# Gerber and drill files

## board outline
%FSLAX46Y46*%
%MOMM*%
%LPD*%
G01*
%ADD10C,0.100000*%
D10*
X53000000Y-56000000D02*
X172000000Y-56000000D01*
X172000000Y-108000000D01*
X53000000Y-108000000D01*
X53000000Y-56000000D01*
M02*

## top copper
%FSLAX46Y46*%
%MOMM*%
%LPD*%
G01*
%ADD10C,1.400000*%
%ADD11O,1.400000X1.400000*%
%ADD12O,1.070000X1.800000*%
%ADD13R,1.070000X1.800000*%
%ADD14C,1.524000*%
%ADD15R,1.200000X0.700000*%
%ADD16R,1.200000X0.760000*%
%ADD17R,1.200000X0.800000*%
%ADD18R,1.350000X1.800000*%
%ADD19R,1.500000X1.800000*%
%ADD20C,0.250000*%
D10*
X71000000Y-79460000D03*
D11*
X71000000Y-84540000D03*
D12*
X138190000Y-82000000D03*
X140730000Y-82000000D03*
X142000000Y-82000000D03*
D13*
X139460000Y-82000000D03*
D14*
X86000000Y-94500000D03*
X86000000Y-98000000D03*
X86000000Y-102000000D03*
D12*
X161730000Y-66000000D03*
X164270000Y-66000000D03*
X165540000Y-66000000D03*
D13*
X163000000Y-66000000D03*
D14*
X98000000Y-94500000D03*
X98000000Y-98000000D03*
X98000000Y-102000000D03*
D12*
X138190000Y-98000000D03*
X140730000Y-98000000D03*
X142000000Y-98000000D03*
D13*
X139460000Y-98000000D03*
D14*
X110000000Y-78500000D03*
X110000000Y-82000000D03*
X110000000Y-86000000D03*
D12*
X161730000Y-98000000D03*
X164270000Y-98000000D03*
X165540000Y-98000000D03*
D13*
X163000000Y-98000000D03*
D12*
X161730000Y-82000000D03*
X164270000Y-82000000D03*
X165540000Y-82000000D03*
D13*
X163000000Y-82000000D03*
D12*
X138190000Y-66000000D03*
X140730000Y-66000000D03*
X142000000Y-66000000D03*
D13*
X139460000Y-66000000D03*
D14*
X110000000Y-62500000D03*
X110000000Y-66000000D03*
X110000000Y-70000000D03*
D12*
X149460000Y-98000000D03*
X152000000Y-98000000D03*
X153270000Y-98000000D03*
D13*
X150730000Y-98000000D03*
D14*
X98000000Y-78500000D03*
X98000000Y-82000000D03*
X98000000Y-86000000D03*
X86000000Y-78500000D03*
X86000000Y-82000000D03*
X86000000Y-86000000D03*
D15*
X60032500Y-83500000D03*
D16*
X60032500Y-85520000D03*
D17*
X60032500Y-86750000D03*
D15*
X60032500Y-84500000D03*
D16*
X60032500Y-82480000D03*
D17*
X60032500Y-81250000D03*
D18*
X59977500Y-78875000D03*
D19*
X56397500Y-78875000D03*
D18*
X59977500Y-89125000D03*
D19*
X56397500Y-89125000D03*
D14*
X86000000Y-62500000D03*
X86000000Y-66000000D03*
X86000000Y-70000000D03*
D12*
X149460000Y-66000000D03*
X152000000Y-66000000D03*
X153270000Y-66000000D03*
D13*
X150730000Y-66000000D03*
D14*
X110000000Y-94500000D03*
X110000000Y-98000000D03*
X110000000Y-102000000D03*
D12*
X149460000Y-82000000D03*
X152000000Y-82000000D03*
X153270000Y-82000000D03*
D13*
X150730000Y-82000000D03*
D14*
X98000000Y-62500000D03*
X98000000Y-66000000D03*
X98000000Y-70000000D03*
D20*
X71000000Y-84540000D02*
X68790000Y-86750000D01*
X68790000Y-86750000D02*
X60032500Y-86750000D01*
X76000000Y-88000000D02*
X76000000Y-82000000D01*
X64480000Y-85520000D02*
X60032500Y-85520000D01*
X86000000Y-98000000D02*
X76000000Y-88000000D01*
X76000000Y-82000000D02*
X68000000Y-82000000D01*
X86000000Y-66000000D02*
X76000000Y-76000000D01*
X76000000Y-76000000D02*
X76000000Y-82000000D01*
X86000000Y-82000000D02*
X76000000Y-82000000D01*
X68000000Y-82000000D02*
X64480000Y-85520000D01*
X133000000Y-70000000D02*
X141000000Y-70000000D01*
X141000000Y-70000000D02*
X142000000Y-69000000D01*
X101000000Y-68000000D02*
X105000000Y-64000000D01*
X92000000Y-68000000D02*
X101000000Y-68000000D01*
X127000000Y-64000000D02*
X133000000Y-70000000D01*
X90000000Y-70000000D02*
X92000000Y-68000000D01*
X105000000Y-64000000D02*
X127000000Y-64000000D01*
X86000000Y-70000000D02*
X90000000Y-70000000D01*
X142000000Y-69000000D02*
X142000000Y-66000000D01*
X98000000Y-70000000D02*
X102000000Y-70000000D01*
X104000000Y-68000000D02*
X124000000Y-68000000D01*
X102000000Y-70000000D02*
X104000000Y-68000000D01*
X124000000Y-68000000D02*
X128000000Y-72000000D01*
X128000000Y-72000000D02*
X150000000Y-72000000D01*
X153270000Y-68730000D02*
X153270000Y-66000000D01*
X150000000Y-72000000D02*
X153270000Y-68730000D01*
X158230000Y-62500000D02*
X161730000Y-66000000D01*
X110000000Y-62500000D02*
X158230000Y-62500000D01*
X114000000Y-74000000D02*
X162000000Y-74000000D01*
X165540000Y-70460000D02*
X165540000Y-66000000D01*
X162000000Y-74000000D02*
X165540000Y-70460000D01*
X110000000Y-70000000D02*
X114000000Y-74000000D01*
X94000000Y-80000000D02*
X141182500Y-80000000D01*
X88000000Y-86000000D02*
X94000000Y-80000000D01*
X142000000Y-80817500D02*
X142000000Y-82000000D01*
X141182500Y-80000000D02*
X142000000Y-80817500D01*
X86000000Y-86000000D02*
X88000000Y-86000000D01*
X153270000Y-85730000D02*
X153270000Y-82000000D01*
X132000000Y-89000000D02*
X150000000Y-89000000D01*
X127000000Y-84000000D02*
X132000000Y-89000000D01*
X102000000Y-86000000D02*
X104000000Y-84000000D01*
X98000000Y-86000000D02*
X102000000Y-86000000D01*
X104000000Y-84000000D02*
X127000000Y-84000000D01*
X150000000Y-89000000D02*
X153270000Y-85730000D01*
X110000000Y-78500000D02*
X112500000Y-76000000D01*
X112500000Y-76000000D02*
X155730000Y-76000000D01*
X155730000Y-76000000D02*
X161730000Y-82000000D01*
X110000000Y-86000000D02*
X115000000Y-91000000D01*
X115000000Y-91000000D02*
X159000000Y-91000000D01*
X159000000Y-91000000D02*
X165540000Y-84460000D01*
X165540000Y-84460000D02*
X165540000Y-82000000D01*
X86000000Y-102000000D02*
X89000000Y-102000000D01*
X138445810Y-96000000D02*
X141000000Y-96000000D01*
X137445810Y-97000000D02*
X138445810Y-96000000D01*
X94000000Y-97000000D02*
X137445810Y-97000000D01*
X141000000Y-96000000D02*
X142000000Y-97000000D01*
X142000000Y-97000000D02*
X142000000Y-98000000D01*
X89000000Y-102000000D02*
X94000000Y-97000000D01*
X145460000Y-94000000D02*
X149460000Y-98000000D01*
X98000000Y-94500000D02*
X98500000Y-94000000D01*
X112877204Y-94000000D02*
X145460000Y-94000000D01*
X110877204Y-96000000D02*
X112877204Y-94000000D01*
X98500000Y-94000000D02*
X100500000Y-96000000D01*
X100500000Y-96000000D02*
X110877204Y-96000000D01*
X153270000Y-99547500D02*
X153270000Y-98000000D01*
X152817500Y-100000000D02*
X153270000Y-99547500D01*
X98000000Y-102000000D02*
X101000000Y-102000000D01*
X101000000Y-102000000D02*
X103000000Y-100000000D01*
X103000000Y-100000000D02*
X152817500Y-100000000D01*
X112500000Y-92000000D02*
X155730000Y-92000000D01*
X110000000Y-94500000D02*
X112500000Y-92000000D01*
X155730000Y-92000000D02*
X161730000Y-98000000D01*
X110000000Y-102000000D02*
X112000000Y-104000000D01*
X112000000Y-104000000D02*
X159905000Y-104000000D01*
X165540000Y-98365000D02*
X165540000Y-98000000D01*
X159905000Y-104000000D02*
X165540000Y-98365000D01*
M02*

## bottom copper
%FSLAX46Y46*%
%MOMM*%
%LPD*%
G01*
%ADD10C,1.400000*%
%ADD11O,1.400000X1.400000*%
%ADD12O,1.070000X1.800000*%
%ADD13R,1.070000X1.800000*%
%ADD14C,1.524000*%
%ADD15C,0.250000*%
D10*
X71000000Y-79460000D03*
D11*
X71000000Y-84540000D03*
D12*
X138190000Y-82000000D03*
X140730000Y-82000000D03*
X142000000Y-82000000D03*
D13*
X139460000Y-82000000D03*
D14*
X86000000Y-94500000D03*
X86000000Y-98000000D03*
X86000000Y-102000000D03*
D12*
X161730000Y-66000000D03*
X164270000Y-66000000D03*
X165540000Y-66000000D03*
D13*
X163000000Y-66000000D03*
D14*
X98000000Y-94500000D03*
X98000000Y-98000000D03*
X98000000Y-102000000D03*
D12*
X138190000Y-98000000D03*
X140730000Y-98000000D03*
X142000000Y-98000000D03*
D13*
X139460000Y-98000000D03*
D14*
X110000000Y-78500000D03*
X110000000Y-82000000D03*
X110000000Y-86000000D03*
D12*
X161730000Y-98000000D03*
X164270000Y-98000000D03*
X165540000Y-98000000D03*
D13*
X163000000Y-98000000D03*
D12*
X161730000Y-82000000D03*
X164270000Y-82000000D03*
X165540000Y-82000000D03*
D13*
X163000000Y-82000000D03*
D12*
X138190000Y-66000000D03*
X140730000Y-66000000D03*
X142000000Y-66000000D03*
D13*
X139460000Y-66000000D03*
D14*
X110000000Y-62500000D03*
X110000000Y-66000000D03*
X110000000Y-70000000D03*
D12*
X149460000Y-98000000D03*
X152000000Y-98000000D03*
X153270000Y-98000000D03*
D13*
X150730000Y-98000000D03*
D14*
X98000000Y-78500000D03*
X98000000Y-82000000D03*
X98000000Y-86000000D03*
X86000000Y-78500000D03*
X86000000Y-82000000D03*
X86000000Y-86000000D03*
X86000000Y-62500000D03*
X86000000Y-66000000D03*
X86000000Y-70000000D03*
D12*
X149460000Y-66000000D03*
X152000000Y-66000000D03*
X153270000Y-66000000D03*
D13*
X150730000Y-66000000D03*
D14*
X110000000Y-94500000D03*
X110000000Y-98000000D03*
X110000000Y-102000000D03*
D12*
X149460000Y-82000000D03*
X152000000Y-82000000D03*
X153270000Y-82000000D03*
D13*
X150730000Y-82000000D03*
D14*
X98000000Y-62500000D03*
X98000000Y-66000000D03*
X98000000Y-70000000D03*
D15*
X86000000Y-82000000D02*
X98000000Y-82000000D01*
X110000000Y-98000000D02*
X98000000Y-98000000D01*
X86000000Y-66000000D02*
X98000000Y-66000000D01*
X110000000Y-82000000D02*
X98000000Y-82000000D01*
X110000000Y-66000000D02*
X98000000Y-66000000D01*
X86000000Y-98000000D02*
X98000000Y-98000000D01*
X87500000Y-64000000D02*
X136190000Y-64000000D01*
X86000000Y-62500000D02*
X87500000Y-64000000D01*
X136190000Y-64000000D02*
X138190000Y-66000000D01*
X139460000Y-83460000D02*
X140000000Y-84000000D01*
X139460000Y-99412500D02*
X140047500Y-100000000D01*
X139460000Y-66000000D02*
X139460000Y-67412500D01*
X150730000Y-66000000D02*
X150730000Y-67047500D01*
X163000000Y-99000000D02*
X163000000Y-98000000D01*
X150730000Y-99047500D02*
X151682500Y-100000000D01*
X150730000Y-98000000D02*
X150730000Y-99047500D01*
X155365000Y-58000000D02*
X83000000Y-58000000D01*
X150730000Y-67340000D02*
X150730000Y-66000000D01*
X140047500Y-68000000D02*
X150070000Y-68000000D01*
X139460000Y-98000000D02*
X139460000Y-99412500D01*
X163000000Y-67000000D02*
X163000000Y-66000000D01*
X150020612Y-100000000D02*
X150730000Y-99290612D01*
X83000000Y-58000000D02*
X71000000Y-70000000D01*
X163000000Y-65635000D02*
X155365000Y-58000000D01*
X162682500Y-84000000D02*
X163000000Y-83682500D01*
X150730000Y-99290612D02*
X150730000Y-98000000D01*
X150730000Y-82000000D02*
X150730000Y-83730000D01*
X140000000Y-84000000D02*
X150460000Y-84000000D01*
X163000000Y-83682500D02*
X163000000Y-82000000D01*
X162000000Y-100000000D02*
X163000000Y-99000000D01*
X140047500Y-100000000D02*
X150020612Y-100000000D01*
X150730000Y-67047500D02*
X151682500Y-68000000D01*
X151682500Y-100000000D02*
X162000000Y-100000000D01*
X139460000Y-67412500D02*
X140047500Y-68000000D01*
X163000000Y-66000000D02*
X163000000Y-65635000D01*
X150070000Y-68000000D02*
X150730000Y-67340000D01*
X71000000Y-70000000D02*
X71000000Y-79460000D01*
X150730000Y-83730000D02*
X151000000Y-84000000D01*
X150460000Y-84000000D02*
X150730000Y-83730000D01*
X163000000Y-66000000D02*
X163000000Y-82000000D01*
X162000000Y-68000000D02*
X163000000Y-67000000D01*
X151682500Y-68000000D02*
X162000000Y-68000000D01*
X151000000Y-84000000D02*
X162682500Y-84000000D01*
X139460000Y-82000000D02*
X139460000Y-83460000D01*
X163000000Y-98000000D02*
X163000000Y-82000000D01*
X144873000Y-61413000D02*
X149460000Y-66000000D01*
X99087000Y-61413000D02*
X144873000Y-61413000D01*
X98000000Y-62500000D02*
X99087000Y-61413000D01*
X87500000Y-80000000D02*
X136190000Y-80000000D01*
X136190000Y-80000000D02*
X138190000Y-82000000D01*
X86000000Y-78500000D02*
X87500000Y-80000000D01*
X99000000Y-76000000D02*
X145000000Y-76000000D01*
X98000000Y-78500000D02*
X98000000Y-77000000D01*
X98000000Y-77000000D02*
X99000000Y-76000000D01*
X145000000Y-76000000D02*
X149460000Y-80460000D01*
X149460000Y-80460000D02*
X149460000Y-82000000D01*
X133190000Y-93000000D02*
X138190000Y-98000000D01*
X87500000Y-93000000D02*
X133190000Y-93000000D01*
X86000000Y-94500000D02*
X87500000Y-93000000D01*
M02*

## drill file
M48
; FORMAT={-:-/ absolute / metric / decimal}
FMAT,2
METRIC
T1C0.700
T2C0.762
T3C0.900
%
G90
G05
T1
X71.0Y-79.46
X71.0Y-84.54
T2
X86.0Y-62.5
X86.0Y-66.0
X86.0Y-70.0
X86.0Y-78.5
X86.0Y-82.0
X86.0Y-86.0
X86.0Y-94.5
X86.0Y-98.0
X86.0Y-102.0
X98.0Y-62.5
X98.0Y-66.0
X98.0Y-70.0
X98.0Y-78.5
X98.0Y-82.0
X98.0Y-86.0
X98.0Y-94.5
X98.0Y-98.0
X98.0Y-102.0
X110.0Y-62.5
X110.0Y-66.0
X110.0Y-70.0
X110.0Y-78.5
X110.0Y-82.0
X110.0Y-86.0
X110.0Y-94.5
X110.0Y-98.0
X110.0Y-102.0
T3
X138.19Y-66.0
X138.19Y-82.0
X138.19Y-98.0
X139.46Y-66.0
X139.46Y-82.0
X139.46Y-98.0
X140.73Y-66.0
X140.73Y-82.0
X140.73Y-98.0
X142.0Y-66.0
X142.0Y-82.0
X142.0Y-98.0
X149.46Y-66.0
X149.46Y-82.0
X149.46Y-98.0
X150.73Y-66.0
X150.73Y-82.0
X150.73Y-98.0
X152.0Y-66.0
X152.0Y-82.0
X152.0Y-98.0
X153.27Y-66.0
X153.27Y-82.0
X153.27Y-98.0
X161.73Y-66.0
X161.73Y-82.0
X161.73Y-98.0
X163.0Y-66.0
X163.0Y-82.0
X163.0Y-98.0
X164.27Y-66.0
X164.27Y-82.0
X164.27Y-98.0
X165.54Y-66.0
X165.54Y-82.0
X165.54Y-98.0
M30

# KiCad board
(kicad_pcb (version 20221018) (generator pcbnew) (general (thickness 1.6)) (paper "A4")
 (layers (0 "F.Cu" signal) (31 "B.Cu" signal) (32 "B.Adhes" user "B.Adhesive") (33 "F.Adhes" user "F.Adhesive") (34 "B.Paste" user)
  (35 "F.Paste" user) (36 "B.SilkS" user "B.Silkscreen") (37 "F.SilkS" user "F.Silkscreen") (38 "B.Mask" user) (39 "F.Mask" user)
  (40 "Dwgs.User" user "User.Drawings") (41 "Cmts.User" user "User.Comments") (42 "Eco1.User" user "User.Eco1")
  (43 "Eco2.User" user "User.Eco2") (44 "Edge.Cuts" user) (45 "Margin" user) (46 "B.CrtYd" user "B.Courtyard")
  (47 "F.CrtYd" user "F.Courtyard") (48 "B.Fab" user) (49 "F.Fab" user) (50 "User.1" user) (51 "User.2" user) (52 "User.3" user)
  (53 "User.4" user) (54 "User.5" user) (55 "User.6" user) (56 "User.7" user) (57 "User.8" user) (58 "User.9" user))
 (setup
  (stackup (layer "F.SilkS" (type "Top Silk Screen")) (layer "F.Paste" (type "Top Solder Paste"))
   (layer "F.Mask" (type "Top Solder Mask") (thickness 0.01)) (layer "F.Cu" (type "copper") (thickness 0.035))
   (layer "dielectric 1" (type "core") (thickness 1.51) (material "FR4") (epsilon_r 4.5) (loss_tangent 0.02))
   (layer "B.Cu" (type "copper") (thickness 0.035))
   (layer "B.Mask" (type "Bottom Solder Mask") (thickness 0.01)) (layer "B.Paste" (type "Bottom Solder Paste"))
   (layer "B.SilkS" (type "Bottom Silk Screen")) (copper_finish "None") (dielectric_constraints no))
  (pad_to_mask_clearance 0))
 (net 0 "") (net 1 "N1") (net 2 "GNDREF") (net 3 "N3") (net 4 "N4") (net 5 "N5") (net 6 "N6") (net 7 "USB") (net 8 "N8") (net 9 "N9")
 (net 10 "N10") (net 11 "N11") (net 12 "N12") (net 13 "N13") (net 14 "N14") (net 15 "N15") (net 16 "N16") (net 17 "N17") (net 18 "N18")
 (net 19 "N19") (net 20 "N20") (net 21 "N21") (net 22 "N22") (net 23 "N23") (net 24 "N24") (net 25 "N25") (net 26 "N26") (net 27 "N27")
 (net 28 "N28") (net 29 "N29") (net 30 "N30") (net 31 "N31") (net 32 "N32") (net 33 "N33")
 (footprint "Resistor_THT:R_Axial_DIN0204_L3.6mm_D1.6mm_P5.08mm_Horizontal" (layer "F.Cu") (at 71 79.46 -90)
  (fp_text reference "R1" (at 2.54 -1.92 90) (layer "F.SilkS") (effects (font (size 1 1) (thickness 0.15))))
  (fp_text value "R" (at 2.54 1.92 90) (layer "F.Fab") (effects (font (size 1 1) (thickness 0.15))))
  (pad "1" thru_hole circle (at 0 0 270) (size 1.4 1.4) (drill 0.7) (layers "*.Cu" "*.Mask") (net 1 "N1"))
  (pad "2" thru_hole oval (at 5.08 0 270) (size 1.4 1.4) (drill 0.7) (layers "*.Cu" "*.Mask") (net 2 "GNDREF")))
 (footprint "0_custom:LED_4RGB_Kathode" (layer "F.Cu") (at 140.095 82)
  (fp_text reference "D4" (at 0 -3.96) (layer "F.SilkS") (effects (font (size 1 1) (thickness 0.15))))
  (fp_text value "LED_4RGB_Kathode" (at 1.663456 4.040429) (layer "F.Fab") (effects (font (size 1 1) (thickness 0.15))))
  (pad "1" thru_hole oval (at -1.905 0) (size 1.07 1.8) (drill 0.9) (layers "*.Cu" "*.Mask") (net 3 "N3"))
  (pad "2" thru_hole oval (at 0.635 0) (size 1.07 1.8) (drill 0.9) (layers "*.Cu" "*.Mask") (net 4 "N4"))
  (pad "3" thru_hole oval (at 1.905 0) (size 1.07 1.8) (drill 0.9) (layers "*.Cu" "*.Mask") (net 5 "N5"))
  (pad "4" thru_hole rect (at -0.635 0) (size 1.07 1.8) (drill 0.9) (layers "*.Cu" "*.Mask") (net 1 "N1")))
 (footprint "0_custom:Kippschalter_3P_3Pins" (layer "F.Cu") (at 86 98 -90)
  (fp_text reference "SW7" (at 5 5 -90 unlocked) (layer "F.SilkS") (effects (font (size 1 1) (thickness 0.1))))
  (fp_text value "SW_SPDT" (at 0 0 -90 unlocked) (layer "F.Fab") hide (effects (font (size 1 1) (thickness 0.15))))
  (pad "1" thru_hole circle (at -3.5 0 270) (size 1.524 1.524) (drill 0.762) (layers "*.Cu" "*.Mask") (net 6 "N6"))
  (pad "2" thru_hole circle (at 0 0 270) (size 1.524 1.524) (drill 0.762) (layers "*.Cu" "*.Mask") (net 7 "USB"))
  (pad "3" thru_hole circle (at 4 0 270) (size 1.524 1.524) (drill 0.762) (layers "*.Cu" "*.Mask") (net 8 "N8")))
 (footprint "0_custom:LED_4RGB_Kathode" (layer "F.Cu") (at 163.635 66)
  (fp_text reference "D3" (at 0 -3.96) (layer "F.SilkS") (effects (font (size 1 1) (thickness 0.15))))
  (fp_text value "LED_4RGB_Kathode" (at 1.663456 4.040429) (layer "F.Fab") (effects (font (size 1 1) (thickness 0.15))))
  (pad "1" thru_hole oval (at -1.905 0) (size 1.07 1.8) (drill 0.9) (layers "*.Cu" "*.Mask") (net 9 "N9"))
  (pad "2" thru_hole oval (at 0.635 0) (size 1.07 1.8) (drill 0.9) (layers "*.Cu" "*.Mask") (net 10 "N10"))
  (pad "3" thru_hole oval (at 1.905 0) (size 1.07 1.8) (drill 0.9) (layers "*.Cu" "*.Mask") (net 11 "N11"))
  (pad "4" thru_hole rect (at -0.635 0) (size 1.07 1.8) (drill 0.9) (layers "*.Cu" "*.Mask") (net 1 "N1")))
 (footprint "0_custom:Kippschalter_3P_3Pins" (layer "F.Cu") (at 98 98 -90)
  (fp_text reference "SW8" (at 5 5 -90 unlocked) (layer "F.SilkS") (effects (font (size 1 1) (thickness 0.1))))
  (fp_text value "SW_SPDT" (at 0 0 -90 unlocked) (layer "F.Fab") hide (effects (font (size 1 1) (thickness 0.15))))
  (pad "1" thru_hole circle (at -3.5 0 270) (size 1.524 1.524) (drill 0.762) (layers "*.Cu" "*.Mask") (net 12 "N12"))
  (pad "2" thru_hole circle (at 0 0 270) (size 1.524 1.524) (drill 0.762) (layers "*.Cu" "*.Mask") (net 7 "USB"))
  (pad "3" thru_hole circle (at 4 0 270) (size 1.524 1.524) (drill 0.762) (layers "*.Cu" "*.Mask") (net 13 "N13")))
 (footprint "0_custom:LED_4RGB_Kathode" (layer "F.Cu") (at 140.095 98)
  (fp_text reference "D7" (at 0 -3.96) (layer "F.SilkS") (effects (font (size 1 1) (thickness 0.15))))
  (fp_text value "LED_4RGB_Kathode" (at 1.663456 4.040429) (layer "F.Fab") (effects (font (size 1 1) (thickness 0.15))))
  (pad "1" thru_hole oval (at -1.905 0) (size 1.07 1.8) (drill 0.9) (layers "*.Cu" "*.Mask") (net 6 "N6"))
  (pad "2" thru_hole oval (at 0.635 0) (size 1.07 1.8) (drill 0.9) (layers "*.Cu" "*.Mask") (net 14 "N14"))
  (pad "3" thru_hole oval (at 1.905 0) (size 1.07 1.8) (drill 0.9) (layers "*.Cu" "*.Mask") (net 8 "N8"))
  (pad "4" thru_hole rect (at -0.635 0) (size 1.07 1.8) (drill 0.9) (layers "*.Cu" "*.Mask") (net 1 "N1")))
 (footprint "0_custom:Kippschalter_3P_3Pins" (layer "F.Cu") (at 110 82 -90)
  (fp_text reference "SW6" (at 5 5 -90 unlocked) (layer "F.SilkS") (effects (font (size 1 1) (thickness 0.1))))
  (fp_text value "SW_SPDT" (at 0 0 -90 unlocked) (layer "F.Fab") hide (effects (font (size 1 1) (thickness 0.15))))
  (pad "1" thru_hole circle (at -3.5 0 270) (size 1.524 1.524) (drill 0.762) (layers "*.Cu" "*.Mask") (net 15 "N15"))
  (pad "2" thru_hole circle (at 0 0 270) (size 1.524 1.524) (drill 0.762) (layers "*.Cu" "*.Mask") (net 7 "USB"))
  (pad "3" thru_hole circle (at 4 0 270) (size 1.524 1.524) (drill 0.762) (layers "*.Cu" "*.Mask") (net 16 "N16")))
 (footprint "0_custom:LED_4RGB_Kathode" (layer "F.Cu") (at 163.635 98)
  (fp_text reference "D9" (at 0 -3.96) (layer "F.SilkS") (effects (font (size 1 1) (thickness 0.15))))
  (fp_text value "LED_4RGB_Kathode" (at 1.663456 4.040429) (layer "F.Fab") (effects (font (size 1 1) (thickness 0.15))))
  (pad "1" thru_hole oval (at -1.905 0) (size 1.07 1.8) (drill 0.9) (layers "*.Cu" "*.Mask") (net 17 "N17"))
  (pad "2" thru_hole oval (at 0.635 0) (size 1.07 1.8) (drill 0.9) (layers "*.Cu" "*.Mask") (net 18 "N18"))
  (pad "3" thru_hole oval (at 1.905 0) (size 1.07 1.8) (drill 0.9) (layers "*.Cu" "*.Mask") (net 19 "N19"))
  (pad "4" thru_hole rect (at -0.635 0) (size 1.07 1.8) (drill 0.9) (layers "*.Cu" "*.Mask") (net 1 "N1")))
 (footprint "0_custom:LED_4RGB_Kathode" (layer "F.Cu") (at 163.635 82)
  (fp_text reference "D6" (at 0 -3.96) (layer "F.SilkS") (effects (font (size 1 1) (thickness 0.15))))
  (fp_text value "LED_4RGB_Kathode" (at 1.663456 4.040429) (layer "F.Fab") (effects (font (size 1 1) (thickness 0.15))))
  (pad "1" thru_hole oval (at -1.905 0) (size 1.07 1.8) (drill 0.9) (layers "*.Cu" "*.Mask") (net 15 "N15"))
  (pad "2" thru_hole oval (at 0.635 0) (size 1.07 1.8) (drill 0.9) (layers "*.Cu" "*.Mask") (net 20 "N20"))
  (pad "3" thru_hole oval (at 1.905 0) (size 1.07 1.8) (drill 0.9) (layers "*.Cu" "*.Mask") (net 16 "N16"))
  (pad "4" thru_hole rect (at -0.635 0) (size 1.07 1.8) (drill 0.9) (layers "*.Cu" "*.Mask") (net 1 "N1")))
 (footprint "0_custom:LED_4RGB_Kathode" (layer "F.Cu") (at 140.095 66)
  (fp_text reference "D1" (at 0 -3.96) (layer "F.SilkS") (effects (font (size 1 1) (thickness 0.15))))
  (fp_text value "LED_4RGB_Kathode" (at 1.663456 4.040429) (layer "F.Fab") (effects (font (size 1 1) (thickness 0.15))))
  (pad "1" thru_hole oval (at -1.905 0) (size 1.07 1.8) (drill 0.9) (layers "*.Cu" "*.Mask") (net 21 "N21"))
  (pad "2" thru_hole oval (at 0.635 0) (size 1.07 1.8) (drill 0.9) (layers "*.Cu" "*.Mask") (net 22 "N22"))
  (pad "3" thru_hole oval (at 1.905 0) (size 1.07 1.8) (drill 0.9) (layers "*.Cu" "*.Mask") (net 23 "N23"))
  (pad "4" thru_hole rect (at -0.635 0) (size 1.07 1.8) (drill 0.9) (layers "*.Cu" "*.Mask") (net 1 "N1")))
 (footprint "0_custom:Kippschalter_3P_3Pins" (layer "F.Cu") (at 110 66 -90)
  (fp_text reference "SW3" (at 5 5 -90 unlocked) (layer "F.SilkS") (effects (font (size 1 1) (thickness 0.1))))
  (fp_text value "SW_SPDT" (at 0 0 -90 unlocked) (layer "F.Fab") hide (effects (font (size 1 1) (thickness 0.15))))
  (pad "1" thru_hole circle (at -3.5 0 270) (size 1.524 1.524) (drill 0.762) (layers "*.Cu" "*.Mask") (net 9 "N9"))
  (pad "2" thru_hole circle (at 0 0 270) (size 1.524 1.524) (drill 0.762) (layers "*.Cu" "*.Mask") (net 7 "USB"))
  (pad "3" thru_hole circle (at 4 0 270) (size 1.524 1.524) (drill 0.762) (layers "*.Cu" "*.Mask") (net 11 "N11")))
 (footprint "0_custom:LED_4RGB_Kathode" (layer "F.Cu") (at 151.365 98)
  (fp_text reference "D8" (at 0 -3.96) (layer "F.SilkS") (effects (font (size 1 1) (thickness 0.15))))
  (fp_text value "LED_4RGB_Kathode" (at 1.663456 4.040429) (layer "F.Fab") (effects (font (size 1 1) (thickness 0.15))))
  (pad "1" thru_hole oval (at -1.905 0) (size 1.07 1.8) (drill 0.9) (layers "*.Cu" "*.Mask") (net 12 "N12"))
  (pad "2" thru_hole oval (at 0.635 0) (size 1.07 1.8) (drill 0.9) (layers "*.Cu" "*.Mask") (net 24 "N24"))
  (pad "3" thru_hole oval (at 1.905 0) (size 1.07 1.8) (drill 0.9) (layers "*.Cu" "*.Mask") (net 13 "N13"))
  (pad "4" thru_hole rect (at -0.635 0) (size 1.07 1.8) (drill 0.9) (layers "*.Cu" "*.Mask") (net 1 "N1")))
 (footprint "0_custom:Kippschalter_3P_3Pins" (layer "F.Cu") (at 98 82 -90)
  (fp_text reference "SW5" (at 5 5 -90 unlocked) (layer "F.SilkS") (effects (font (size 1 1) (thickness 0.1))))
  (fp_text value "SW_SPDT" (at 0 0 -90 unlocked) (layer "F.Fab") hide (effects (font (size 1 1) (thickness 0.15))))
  (pad "1" thru_hole circle (at -3.5 0 270) (size 1.524 1.524) (drill 0.762) (layers "*.Cu" "*.Mask") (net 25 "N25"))
  (pad "2" thru_hole circle (at 0 0 270) (size 1.524 1.524) (drill 0.762) (layers "*.Cu" "*.Mask") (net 7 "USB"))
  (pad "3" thru_hole circle (at 4 0 270) (size 1.524 1.524) (drill 0.762) (layers "*.Cu" "*.Mask") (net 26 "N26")))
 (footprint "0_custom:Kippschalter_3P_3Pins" (layer "F.Cu") (at 86 82 -90)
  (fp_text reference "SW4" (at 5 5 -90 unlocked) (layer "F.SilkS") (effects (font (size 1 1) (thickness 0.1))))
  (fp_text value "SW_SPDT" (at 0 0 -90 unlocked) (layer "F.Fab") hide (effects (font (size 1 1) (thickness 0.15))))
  (pad "1" thru_hole circle (at -3.5 0 270) (size 1.524 1.524) (drill 0.762) (layers "*.Cu" "*.Mask") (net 3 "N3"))
  (pad "2" thru_hole circle (at 0 0 270) (size 1.524 1.524) (drill 0.762) (layers "*.Cu" "*.Mask") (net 7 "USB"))
  (pad "3" thru_hole circle (at 4 0 270) (size 1.524 1.524) (drill 0.762) (layers "*.Cu" "*.Mask") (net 5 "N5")))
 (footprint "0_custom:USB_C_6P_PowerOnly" (layer "F.Cu") (at 57 84 -90)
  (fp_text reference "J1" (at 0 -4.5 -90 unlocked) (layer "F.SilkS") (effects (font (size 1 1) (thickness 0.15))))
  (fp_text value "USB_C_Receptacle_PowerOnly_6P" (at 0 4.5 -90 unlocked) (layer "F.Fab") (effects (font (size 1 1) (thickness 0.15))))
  (pad "A5" smd rect (at -0.5 -3.0325 270) (size 0.7 1.2) (layers "F.Cu" "F.Paste" "F.Mask") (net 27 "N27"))
  (pad "A9" smd rect (at 1.52 -3.0325 90) (size 0.76 1.2) (layers "F.Cu" "F.Paste" "F.Mask") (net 7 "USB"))
  (pad "A12" smd rect (at 2.75 -3.0325 90) (size 0.8 1.2) (layers "F.Cu" "F.Paste" "F.Mask") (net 2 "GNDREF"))
  (pad "B5" smd rect (at 0.5 -3.0325 90) (size 0.7 1.2) (layers "F.Cu" "F.Paste" "F.Mask") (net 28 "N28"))
  (pad "B9" smd rect (at -1.52 -3.0325 270) (size 0.76 1.2) (layers "F.Cu" "F.Paste" "F.Mask") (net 7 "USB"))
  (pad "B12" smd rect (at -2.75 -3.0325 270) (size 0.8 1.2) (layers "F.Cu" "F.Paste" "F.Mask") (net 2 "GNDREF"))
  (pad "S1" smd rect (at -5.125 -2.9775 270) (size 1.8 1.35) (layers "F.Cu" "F.Paste" "F.Mask") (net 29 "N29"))
  (pad "S1" smd rect (at -5.125 0.6025 270) (size 1.8 1.5) (layers "F.Cu" "F.Paste" "F.Mask") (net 29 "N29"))
  (pad "S1" smd rect (at 5.125 -2.9775 270) (size 1.8 1.35) (layers "F.Cu" "F.Paste" "F.Mask") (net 29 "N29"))
  (pad "S1" smd rect (at 5.125 0.6025 270) (size 1.8 1.5) (layers "F.Cu" "F.Paste" "F.Mask") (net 29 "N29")))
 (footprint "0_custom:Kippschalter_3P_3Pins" (layer "F.Cu") (at 86 66 -90)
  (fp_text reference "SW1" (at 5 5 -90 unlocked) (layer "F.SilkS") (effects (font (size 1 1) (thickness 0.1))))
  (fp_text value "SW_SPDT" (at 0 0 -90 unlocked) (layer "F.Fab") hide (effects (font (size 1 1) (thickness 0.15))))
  (pad "1" thru_hole circle (at -3.5 0 270) (size 1.524 1.524) (drill 0.762) (layers "*.Cu" "*.Mask") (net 21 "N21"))
  (pad "2" thru_hole circle (at 0 0 270) (size 1.524 1.524) (drill 0.762) (layers "*.Cu" "*.Mask") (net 7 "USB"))
  (pad "3" thru_hole circle (at 4 0 270) (size 1.524 1.524) (drill 0.762) (layers "*.Cu" "*.Mask") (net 23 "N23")))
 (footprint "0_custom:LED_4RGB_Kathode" (layer "F.Cu") (at 151.365 66)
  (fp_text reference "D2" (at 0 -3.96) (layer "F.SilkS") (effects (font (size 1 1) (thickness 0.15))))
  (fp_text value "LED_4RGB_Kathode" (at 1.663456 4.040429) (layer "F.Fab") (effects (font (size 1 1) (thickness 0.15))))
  (pad "1" thru_hole oval (at -1.905 0) (size 1.07 1.8) (drill 0.9) (layers "*.Cu" "*.Mask") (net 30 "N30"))
  (pad "2" thru_hole oval (at 0.635 0) (size 1.07 1.8) (drill 0.9) (layers "*.Cu" "*.Mask") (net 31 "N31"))
  (pad "3" thru_hole oval (at 1.905 0) (size 1.07 1.8) (drill 0.9) (layers "*.Cu" "*.Mask") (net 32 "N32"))
  (pad "4" thru_hole rect (at -0.635 0) (size 1.07 1.8) (drill 0.9) (layers "*.Cu" "*.Mask") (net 1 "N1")))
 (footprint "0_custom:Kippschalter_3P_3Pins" (layer "F.Cu") (at 110 98 -90)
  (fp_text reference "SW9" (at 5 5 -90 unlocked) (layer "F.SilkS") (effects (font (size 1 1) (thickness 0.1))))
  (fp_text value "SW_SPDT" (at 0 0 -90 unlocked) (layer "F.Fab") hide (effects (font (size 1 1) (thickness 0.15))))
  (pad "1" thru_hole circle (at -3.5 0 270) (size 1.524 1.524) (drill 0.762) (layers "*.Cu" "*.Mask") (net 17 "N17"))
  (pad "2" thru_hole circle (at 0 0 270) (size 1.524 1.524) (drill 0.762) (layers "*.Cu" "*.Mask") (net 7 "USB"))
  (pad "3" thru_hole circle (at 4 0 270) (size 1.524 1.524) (drill 0.762) (layers "*.Cu" "*.Mask") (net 19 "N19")))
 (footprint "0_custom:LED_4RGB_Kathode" (layer "F.Cu") (at 151.365 82)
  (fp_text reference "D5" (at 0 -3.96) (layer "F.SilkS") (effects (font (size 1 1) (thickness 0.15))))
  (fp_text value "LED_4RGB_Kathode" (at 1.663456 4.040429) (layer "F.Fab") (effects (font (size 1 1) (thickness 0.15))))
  (pad "1" thru_hole oval (at -1.905 0) (size 1.07 1.8) (drill 0.9) (layers "*.Cu" "*.Mask") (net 25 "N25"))
  (pad "2" thru_hole oval (at 0.635 0) (size 1.07 1.8) (drill 0.9) (layers "*.Cu" "*.Mask") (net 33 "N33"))
  (pad "3" thru_hole oval (at 1.905 0) (size 1.07 1.8) (drill 0.9) (layers "*.Cu" "*.Mask") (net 26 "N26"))
  (pad "4" thru_hole rect (at -0.635 0) (size 1.07 1.8) (drill 0.9) (layers "*.Cu" "*.Mask") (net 1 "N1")))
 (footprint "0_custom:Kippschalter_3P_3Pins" (layer "F.Cu") (at 98 66 -90)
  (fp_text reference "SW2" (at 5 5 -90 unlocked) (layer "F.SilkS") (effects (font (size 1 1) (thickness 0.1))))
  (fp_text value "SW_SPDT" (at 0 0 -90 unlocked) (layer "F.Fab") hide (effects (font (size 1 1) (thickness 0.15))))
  (pad "1" thru_hole circle (at -3.5 0 270) (size 1.524 1.524) (drill 0.762) (layers "*.Cu" "*.Mask") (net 30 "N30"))
  (pad "2" thru_hole circle (at 0 0 270) (size 1.524 1.524) (drill 0.762) (layers "*.Cu" "*.Mask") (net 7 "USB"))
  (pad "3" thru_hole circle (at 4 0 270) (size 1.524 1.524) (drill 0.762) (layers "*.Cu" "*.Mask") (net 32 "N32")))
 (gr_rect (start 53 56) (end 172 108) (stroke (width 0.1) (type default)) (fill none) (layer "Edge.Cuts"))
 (segment (start 71 84.54) (end 68.79 86.75) (width 0.25) (layer "F.Cu") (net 2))
 (segment (start 68.79 86.75) (end 60.0325 86.75) (width 0.25) (layer "F.Cu") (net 2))
 (segment (start 76 88) (end 76 82) (width 0.25) (layer "F.Cu") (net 7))
 (segment (start 64.48 85.52) (end 60.0325 85.52) (width 0.25) (layer "F.Cu") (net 7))
 (segment (start 86 98) (end 76 88) (width 0.25) (layer "F.Cu") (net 7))
 (segment (start 76 82) (end 68 82) (width 0.25) (layer "F.Cu") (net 7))
 (segment (start 86 66) (end 76 76) (width 0.25) (layer "F.Cu") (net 7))
 (segment (start 76 76) (end 76 82) (width 0.25) (layer "F.Cu") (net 7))
 (segment (start 86 82) (end 76 82) (width 0.25) (layer "F.Cu") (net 7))
 (segment (start 68 82) (end 64.48 85.52) (width 0.25) (layer "F.Cu") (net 7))
 (segment (start 86 82) (end 98 82) (width 0.25) (layer "B.Cu") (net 7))
 (segment (start 110 98) (end 98 98) (width 0.25) (layer "B.Cu") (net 7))
 (segment (start 86 66) (end 98 66) (width 0.25) (layer "B.Cu") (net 7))
 (segment (start 110 82) (end 98 82) (width 0.25) (layer "B.Cu") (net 7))
 (segment (start 110 66) (end 98 66) (width 0.25) (layer "B.Cu") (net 7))
 (segment (start 86 98) (end 98 98) (width 0.25) (layer "B.Cu") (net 7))
 (segment (start 87.5 64) (end 136.19 64) (width 0.25) (layer "B.Cu") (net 21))
 (segment (start 86 62.5) (end 87.5 64) (width 0.25) (layer "B.Cu") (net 21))
 (segment (start 136.19 64) (end 138.19 66) (width 0.25) (layer "B.Cu") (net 21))
 (segment (start 133 70) (end 141 70) (width 0.25) (layer "F.Cu") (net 23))
 (segment (start 141 70) (end 142 69) (width 0.25) (layer "F.Cu") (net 23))
 (segment (start 101 68) (end 105 64) (width 0.25) (layer "F.Cu") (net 23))
 (segment (start 92 68) (end 101 68) (width 0.25) (layer "F.Cu") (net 23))
 (segment (start 127 64) (end 133 70) (width 0.25) (layer "F.Cu") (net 23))
 (segment (start 90 70) (end 92 68) (width 0.25) (layer "F.Cu") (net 23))
 (segment (start 105 64) (end 127 64) (width 0.25) (layer "F.Cu") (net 23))
 (segment (start 86 70) (end 90 70) (width 0.25) (layer "F.Cu") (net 23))
 (segment (start 142 69) (end 142 66) (width 0.25) (layer "F.Cu") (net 23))
 (segment (start 139.46 83.46) (end 140 84) (width 0.25) (layer "B.Cu") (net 1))
 (segment (start 139.46 99.4125) (end 140.0475 100) (width 0.25) (layer "B.Cu") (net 1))
 (segment (start 139.46 66) (end 139.46 67.4125) (width 0.25) (layer "B.Cu") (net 1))
 (segment (start 150.73 66) (end 150.73 67.0475) (width 0.25) (layer "B.Cu") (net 1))
 (segment (start 163 99) (end 163 98) (width 0.25) (layer "B.Cu") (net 1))
 (segment (start 150.73 99.0475) (end 151.6825 100) (width 0.25) (layer "B.Cu") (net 1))
 (segment (start 150.73 98) (end 150.73 99.0475) (width 0.25) (layer "B.Cu") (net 1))
 (segment (start 155.365 58) (end 83 58) (width 0.25) (layer "B.Cu") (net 1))
 (segment (start 150.73 67.34) (end 150.73 66) (width 0.25) (layer "B.Cu") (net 1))
 (segment (start 140.0475 68) (end 150.07 68) (width 0.25) (layer "B.Cu") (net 1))
 (segment (start 139.46 98) (end 139.46 99.4125) (width 0.25) (layer "B.Cu") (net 1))
 (segment (start 163 67) (end 163 66) (width 0.25) (layer "B.Cu") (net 1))
 (segment (start 150.020612 100) (end 150.73 99.290612) (width 0.25) (layer "B.Cu") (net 1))
 (segment (start 83 58) (end 71 70) (width 0.25) (layer "B.Cu") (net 1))
 (segment (start 163 65.635) (end 155.365 58) (width 0.25) (layer "B.Cu") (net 1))
 (segment (start 162.6825 84) (end 163 83.6825) (width 0.25) (layer "B.Cu") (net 1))
 (segment (start 150.73 99.290612) (end 150.73 98) (width 0.25) (layer "B.Cu") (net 1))
 (segment (start 150.73 82) (end 150.73 83.73) (width 0.25) (layer "B.Cu") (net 1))
 (segment (start 140 84) (end 150.46 84) (width 0.25) (layer "B.Cu") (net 1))
 (segment (start 163 83.6825) (end 163 82) (width 0.25) (layer "B.Cu") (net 1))
 (segment (start 162 100) (end 163 99) (width 0.25) (layer "B.Cu") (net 1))
 (segment (start 140.0475 100) (end 150.020612 100) (width 0.25) (layer "B.Cu") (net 1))
 (segment (start 150.73 67.0475) (end 151.6825 68) (width 0.25) (layer "B.Cu") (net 1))
 (segment (start 151.6825 100) (end 162 100) (width 0.25) (layer "B.Cu") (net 1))
 (segment (start 139.46 67.4125) (end 140.0475 68) (width 0.25) (layer "B.Cu") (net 1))
 (segment (start 163 66) (end 163 65.635) (width 0.25) (layer "B.Cu") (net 1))
 (segment (start 150.07 68) (end 150.73 67.34) (width 0.25) (layer "B.Cu") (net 1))
 (segment (start 71 70) (end 71 79.46) (width 0.25) (layer "B.Cu") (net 1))
 (segment (start 150.73 83.73) (end 151 84) (width 0.25) (layer "B.Cu") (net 1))
 (segment (start 150.46 84) (end 150.73 83.73) (width 0.25) (layer "B.Cu") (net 1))
 (segment (start 163 66) (end 163 82) (width 0.25) (layer "B.Cu") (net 1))
 (segment (start 162 68) (end 163 67) (width 0.25) (layer "B.Cu") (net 1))
 (segment (start 151.6825 68) (end 162 68) (width 0.25) (layer "B.Cu") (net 1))
 (segment (start 151 84) (end 162.6825 84) (width 0.25) (layer "B.Cu") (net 1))
 (segment (start 139.46 82) (end 139.46 83.46) (width 0.25) (layer "B.Cu") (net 1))
 (segment (start 163 98) (end 163 82) (width 0.25) (layer "B.Cu") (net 1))
 (segment (start 144.873 61.413) (end 149.46 66) (width 0.25) (layer "B.Cu") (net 30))
 (segment (start 99.087 61.413) (end 144.873 61.413) (width 0.25) (layer "B.Cu") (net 30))
 (segment (start 98 62.5) (end 99.087 61.413) (width 0.25) (layer "B.Cu") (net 30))
 (segment (start 98 70) (end 102 70) (width 0.25) (layer "F.Cu") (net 32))
 (segment (start 104 68) (end 124 68) (width 0.25) (layer "F.Cu") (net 32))
 (segment (start 102 70) (end 104 68) (width 0.25) (layer "F.Cu") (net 32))
 (segment (start 124 68) (end 128 72) (width 0.25) (layer "F.Cu") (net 32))
 (segment (start 128 72) (end 150 72) (width 0.25) (layer "F.Cu") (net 32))
 (segment (start 153.27 68.73) (end 153.27 66) (width 0.25) (layer "F.Cu") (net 32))
 (segment (start 150 72) (end 153.27 68.73) (width 0.25) (layer "F.Cu") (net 32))
 (segment (start 158.23 62.5) (end 161.73 66) (width 0.25) (layer "F.Cu") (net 9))
 (segment (start 110 62.5) (end 158.23 62.5) (width 0.25) (layer "F.Cu") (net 9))
 (segment (start 114 74) (end 162 74) (width 0.25) (layer "F.Cu") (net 11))
 (segment (start 165.54 70.46) (end 165.54 66) (width 0.25) (layer "F.Cu") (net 11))
 (segment (start 162 74) (end 165.54 70.46) (width 0.25) (layer "F.Cu") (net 11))
 (segment (start 110 70) (end 114 74) (width 0.25) (layer "F.Cu") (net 11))
 (segment (start 87.5 80) (end 136.19 80) (width 0.25) (layer "B.Cu") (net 3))
 (segment (start 136.19 80) (end 138.19 82) (width 0.25) (layer "B.Cu") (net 3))
 (segment (start 86 78.5) (end 87.5 80) (width 0.25) (layer "B.Cu") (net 3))
 (segment (start 94 80) (end 141.1825 80) (width 0.25) (layer "F.Cu") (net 5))
 (segment (start 88 86) (end 94 80) (width 0.25) (layer "F.Cu") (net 5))
 (segment (start 142 80.8175) (end 142 82) (width 0.25) (layer "F.Cu") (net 5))
 (segment (start 141.1825 80) (end 142 80.8175) (width 0.25) (layer "F.Cu") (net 5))
 (segment (start 86 86) (end 88 86) (width 0.25) (layer "F.Cu") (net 5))
 (segment (start 99 76) (end 145 76) (width 0.25) (layer "B.Cu") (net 25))
 (segment (start 98 78.5) (end 98 77) (width 0.25) (layer "B.Cu") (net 25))
 (segment (start 98 77) (end 99 76) (width 0.25) (layer "B.Cu") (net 25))
 (segment (start 145 76) (end 149.46 80.46) (width 0.25) (layer "B.Cu") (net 25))
 (segment (start 149.46 80.46) (end 149.46 82) (width 0.25) (layer "B.Cu") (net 25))
 (segment (start 153.27 85.73) (end 153.27 82) (width 0.25) (layer "F.Cu") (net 26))
 (segment (start 132 89) (end 150 89) (width 0.25) (layer "F.Cu") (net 26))
 (segment (start 127 84) (end 132 89) (width 0.25) (layer "F.Cu") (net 26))
 (segment (start 102 86) (end 104 84) (width 0.25) (layer "F.Cu") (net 26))
 (segment (start 98 86) (end 102 86) (width 0.25) (layer "F.Cu") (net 26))
 (segment (start 104 84) (end 127 84) (width 0.25) (layer "F.Cu") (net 26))
 (segment (start 150 89) (end 153.27 85.73) (width 0.25) (layer "F.Cu") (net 26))
 (segment (start 110 78.5) (end 112.5 76) (width 0.25) (layer "F.Cu") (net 15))
 (segment (start 112.5 76) (end 155.73 76) (width 0.25) (layer "F.Cu") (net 15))
 (segment (start 155.73 76) (end 161.73 82) (width 0.25) (layer "F.Cu") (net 15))
 (segment (start 110 86) (end 115 91) (width 0.25) (layer "F.Cu") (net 16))
 (segment (start 115 91) (end 159 91) (width 0.25) (layer "F.Cu") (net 16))
 (segment (start 159 91) (end 165.54 84.46) (width 0.25) (layer "F.Cu") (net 16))
 (segment (start 165.54 84.46) (end 165.54 82) (width 0.25) (layer "F.Cu") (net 16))
 (segment (start 133.19 93) (end 138.19 98) (width 0.25) (layer "B.Cu") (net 6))
 (segment (start 87.5 93) (end 133.19 93) (width 0.25) (layer "B.Cu") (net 6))
 (segment (start 86 94.5) (end 87.5 93) (width 0.25) (layer "B.Cu") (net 6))
 (segment (start 86 102) (end 89 102) (width 0.25) (layer "F.Cu") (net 8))
 (segment (start 138.44581 96) (end 141 96) (width 0.25) (layer "F.Cu") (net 8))
 (segment (start 137.44581 97) (end 138.44581 96) (width 0.25) (layer "F.Cu") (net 8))
 (segment (start 94 97) (end 137.44581 97) (width 0.25) (layer "F.Cu") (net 8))
 (segment (start 141 96) (end 142 97) (width 0.25) (layer "F.Cu") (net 8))
 (segment (start 142 97) (end 142 98) (width 0.25) (layer "F.Cu") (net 8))
 (segment (start 89 102) (end 94 97) (width 0.25) (layer "F.Cu") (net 8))
 (segment (start 145.46 94) (end 149.46 98) (width 0.25) (layer "F.Cu") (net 12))
 (segment (start 98 94.5) (end 98.5 94) (width 0.25) (layer "F.Cu") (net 12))
 (segment (start 112.877204 94) (end 145.46 94) (width 0.25) (layer "F.Cu") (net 12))
 (segment (start 110.877204 96) (end 112.877204 94) (width 0.25) (layer "F.Cu") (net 12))
 (segment (start 98.5 94) (end 100.5 96) (width 0.25) (layer "F.Cu") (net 12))
 (segment (start 100.5 96) (end 110.877204 96) (width 0.25) (layer "F.Cu") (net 12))
 (segment (start 153.27 99.5475) (end 153.27 98) (width 0.25) (layer "F.Cu") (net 13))
 (segment (start 152.8175 100) (end 153.27 99.5475) (width 0.25) (layer "F.Cu") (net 13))
 (segment (start 98 102) (end 101 102) (width 0.25) (layer "F.Cu") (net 13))
 (segment (start 101 102) (end 103 100) (width 0.25) (layer "F.Cu") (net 13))
 (segment (start 103 100) (end 152.8175 100) (width 0.25) (layer "F.Cu") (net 13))
 (segment (start 112.5 92) (end 155.73 92) (width 0.25) (layer "F.Cu") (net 17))
 (segment (start 110 94.5) (end 112.5 92) (width 0.25) (layer "F.Cu") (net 17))
 (segment (start 155.73 92) (end 161.73 98) (width 0.25) (layer "F.Cu") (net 17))
 (segment (start 110 102) (end 112 104) (width 0.25) (layer "F.Cu") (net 19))
 (segment (start 112 104) (end 159.905 104) (width 0.25) (layer "F.Cu") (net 19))
 (segment (start 165.54 98.365) (end 165.54 98) (width 0.25) (layer "F.Cu") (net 19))
 (segment (start 159.905 104) (end 165.54 98.365) (width 0.25) (layer "F.Cu") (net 19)))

